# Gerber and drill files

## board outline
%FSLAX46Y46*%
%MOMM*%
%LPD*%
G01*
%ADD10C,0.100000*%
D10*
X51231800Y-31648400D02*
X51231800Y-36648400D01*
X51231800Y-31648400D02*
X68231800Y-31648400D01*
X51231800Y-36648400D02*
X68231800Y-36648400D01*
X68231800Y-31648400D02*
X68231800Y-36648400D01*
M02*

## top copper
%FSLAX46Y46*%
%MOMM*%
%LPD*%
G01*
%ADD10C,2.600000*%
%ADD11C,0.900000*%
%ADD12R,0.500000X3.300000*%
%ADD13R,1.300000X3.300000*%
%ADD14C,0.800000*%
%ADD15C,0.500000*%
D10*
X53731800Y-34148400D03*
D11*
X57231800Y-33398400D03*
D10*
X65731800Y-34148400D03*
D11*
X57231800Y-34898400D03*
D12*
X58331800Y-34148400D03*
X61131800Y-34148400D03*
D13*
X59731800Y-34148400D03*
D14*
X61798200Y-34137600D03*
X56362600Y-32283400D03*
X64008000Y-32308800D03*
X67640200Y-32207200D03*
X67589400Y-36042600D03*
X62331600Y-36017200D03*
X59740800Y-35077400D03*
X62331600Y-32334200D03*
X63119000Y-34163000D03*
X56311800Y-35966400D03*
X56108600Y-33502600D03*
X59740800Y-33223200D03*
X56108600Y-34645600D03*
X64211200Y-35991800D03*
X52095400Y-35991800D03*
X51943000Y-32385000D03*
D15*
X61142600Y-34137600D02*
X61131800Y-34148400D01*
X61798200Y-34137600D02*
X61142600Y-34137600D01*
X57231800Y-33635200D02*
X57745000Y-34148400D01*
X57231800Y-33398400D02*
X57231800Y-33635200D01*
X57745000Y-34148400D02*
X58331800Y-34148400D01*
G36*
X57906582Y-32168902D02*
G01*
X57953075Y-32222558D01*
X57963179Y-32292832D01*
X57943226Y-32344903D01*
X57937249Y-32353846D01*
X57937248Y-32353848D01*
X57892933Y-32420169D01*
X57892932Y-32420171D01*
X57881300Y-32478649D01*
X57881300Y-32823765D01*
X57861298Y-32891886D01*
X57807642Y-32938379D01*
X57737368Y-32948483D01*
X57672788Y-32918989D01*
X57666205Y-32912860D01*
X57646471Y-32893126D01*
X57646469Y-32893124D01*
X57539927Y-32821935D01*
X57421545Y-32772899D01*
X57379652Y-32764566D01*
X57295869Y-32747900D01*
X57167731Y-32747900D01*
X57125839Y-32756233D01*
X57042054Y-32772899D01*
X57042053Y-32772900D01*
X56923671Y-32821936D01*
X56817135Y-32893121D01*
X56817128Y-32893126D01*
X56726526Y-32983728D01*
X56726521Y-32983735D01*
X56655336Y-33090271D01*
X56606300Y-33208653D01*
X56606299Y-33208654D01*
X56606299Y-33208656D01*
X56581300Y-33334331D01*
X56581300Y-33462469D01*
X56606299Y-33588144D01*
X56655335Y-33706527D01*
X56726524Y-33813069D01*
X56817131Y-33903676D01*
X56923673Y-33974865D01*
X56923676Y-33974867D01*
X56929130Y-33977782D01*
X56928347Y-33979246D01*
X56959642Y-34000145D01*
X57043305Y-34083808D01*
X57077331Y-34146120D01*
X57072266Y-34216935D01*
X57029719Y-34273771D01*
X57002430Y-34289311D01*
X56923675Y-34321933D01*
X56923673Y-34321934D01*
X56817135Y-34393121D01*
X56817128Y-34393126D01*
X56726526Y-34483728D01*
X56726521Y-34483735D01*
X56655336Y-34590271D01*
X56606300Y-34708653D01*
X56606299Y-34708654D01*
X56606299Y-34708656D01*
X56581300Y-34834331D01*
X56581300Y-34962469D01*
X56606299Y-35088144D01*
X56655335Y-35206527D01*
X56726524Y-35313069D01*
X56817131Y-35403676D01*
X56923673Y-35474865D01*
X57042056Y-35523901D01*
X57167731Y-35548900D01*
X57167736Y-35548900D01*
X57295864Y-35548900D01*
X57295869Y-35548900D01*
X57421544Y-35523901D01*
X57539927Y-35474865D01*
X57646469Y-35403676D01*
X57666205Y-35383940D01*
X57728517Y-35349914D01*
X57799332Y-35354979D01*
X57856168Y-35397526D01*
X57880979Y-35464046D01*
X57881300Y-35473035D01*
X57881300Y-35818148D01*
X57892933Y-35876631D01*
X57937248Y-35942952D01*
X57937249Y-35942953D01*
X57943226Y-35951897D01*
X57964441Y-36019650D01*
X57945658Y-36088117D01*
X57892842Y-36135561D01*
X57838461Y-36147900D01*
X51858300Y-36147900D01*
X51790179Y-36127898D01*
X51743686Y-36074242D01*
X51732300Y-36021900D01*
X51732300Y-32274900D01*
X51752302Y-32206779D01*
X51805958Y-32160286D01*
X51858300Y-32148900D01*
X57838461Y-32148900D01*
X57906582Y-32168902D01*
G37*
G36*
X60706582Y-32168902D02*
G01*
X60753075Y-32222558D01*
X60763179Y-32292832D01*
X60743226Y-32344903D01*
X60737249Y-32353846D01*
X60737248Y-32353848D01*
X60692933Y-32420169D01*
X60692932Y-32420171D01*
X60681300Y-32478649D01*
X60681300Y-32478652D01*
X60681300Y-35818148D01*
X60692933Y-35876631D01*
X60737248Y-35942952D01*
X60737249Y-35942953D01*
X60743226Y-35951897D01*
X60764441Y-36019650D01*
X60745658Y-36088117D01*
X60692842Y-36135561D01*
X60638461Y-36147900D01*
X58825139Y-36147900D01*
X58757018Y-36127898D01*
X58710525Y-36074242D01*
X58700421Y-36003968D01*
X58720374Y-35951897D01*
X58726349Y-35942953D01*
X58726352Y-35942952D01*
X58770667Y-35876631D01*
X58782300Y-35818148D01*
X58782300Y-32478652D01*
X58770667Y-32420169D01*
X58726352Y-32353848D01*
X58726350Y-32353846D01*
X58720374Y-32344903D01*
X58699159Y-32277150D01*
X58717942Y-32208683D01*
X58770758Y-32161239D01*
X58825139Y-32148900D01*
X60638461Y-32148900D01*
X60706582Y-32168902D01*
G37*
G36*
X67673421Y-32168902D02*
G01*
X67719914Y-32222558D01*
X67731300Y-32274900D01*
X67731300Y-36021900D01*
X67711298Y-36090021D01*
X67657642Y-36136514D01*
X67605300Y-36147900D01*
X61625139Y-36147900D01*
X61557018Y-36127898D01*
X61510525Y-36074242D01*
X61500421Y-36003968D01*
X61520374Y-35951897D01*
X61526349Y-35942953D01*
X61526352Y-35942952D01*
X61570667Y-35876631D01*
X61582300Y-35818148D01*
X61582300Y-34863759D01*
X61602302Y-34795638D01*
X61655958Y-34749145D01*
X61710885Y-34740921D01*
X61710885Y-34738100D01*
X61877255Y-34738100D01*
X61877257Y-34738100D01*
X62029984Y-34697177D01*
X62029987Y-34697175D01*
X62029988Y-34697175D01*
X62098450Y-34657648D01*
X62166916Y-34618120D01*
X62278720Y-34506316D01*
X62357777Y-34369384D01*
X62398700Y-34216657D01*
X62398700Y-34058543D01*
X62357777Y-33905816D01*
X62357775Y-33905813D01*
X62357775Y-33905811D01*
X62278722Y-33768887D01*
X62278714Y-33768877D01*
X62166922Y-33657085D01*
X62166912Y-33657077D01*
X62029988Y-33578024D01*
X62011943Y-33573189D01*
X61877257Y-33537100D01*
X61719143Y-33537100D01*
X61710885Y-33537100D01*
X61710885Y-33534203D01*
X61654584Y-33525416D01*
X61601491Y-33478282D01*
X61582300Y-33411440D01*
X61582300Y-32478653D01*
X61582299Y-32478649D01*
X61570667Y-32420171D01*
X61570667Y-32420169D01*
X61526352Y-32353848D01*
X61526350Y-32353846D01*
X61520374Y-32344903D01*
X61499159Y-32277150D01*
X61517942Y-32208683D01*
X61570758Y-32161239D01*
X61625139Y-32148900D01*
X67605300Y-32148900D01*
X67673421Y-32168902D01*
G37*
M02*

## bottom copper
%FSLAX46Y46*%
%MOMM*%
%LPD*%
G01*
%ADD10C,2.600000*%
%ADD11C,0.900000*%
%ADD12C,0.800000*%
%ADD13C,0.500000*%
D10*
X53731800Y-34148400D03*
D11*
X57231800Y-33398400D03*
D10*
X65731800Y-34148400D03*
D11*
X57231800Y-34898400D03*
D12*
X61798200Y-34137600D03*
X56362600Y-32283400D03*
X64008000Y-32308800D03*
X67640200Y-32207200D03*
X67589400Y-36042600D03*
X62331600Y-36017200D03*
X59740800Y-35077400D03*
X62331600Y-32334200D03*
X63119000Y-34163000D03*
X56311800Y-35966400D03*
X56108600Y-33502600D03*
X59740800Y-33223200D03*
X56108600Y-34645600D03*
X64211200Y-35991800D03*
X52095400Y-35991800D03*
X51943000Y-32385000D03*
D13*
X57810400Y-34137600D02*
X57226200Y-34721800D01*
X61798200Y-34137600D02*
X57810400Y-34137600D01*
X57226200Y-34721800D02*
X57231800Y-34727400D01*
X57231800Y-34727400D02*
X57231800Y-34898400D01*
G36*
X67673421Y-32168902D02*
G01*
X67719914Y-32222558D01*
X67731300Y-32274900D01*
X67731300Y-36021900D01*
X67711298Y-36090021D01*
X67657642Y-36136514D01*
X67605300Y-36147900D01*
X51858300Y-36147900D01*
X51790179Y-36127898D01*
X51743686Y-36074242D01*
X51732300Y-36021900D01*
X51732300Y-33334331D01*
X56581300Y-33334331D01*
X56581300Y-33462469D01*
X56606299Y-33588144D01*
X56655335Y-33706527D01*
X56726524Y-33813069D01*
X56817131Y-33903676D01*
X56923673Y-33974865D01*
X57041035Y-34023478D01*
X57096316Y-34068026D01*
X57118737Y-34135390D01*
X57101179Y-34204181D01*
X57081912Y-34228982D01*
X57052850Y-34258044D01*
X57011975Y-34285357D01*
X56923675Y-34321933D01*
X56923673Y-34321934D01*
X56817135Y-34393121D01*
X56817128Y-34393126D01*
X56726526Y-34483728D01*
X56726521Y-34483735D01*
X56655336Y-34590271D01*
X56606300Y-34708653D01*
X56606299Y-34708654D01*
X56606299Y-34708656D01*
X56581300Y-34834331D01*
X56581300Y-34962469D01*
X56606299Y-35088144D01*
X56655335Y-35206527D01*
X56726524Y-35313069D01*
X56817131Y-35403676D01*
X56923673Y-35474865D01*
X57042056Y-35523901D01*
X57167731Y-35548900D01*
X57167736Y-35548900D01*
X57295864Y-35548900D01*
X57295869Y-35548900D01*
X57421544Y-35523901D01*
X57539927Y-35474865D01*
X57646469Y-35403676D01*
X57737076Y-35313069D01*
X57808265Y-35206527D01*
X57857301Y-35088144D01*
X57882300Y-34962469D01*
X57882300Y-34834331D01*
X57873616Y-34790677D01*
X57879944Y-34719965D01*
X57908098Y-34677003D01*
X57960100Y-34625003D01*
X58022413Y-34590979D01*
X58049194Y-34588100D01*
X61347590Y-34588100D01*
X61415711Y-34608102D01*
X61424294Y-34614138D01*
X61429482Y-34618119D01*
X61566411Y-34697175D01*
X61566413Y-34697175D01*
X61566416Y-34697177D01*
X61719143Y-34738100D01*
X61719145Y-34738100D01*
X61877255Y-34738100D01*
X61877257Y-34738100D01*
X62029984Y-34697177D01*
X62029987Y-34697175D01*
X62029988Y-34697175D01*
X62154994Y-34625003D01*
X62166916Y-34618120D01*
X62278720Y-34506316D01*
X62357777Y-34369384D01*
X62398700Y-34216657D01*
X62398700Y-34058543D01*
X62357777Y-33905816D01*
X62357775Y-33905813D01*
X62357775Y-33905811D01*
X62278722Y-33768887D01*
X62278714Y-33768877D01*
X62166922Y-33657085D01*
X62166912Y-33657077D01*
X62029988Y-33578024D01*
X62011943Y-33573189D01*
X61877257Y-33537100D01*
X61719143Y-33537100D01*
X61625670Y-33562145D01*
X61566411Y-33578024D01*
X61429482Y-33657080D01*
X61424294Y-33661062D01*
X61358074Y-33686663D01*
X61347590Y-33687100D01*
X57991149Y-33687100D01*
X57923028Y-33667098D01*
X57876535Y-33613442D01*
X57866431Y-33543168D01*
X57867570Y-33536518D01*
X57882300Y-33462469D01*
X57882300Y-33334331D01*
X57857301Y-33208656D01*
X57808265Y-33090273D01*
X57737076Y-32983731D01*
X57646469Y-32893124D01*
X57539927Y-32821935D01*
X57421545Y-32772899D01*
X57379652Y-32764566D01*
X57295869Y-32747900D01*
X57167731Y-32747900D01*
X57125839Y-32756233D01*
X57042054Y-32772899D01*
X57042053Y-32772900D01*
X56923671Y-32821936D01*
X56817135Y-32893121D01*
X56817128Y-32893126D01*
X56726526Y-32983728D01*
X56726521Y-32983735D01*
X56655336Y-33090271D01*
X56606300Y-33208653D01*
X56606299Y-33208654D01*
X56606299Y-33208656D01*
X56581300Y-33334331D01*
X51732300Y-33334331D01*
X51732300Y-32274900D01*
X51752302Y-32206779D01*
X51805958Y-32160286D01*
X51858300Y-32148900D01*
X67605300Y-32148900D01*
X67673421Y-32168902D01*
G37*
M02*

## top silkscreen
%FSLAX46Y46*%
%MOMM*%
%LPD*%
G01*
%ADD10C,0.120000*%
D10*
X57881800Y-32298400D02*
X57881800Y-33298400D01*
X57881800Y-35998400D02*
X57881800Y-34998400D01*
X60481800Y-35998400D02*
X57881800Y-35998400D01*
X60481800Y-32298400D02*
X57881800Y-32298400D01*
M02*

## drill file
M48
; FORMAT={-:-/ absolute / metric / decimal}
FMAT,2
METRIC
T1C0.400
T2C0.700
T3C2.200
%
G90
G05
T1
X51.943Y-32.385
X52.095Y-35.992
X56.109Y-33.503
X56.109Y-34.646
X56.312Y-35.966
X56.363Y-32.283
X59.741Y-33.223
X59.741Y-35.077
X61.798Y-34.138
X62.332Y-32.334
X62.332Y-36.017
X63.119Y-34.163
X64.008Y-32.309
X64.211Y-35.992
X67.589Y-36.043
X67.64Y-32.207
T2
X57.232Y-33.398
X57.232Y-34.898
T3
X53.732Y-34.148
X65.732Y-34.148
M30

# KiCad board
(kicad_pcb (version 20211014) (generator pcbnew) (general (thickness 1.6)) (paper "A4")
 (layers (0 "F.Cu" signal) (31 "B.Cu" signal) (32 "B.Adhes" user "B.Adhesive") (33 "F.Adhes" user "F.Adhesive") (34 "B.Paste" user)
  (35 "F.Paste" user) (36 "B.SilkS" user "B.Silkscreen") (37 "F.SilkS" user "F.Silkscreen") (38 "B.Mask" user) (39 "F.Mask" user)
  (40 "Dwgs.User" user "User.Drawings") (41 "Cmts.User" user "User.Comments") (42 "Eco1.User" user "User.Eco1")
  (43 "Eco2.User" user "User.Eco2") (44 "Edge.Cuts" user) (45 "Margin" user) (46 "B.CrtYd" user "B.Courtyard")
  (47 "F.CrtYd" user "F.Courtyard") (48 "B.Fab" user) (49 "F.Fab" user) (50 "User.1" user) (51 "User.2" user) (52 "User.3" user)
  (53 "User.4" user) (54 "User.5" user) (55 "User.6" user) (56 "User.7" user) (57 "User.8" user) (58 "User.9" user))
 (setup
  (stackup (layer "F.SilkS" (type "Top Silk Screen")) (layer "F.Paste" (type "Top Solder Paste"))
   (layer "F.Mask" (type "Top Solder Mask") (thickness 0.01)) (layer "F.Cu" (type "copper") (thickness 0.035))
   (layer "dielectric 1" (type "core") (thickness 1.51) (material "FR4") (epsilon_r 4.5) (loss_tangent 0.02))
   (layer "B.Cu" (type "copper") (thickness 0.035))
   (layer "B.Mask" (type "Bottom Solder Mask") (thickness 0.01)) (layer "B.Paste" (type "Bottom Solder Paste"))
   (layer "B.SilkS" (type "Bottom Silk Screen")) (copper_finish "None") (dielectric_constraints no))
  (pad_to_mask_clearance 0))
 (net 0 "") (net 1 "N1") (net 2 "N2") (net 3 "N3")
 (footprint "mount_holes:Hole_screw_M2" (layer "F.Cu") (at 53.7318 34.1484)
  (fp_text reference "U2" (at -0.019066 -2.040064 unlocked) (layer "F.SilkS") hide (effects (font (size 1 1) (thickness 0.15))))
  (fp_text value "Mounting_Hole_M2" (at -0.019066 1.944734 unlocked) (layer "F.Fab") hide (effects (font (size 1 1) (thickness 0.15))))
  (pad "1" thru_hole circle (at 0 0) (size 2.6 2.6) (drill 2.2) (layers *.Cu *.Mask) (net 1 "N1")))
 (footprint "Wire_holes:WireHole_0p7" (layer "F.Cu") (at 57.2318 33.3984)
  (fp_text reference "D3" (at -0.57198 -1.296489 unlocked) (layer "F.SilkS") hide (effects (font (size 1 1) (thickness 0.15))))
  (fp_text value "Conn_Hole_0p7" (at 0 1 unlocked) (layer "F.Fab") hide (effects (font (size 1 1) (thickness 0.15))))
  (pad "1" thru_hole circle (at 0 0) (size 0.9 0.9) (drill 0.7) (layers *.Cu *.Mask) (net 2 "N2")))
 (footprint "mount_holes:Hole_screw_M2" (layer "F.Cu") (at 65.7318 34.1484)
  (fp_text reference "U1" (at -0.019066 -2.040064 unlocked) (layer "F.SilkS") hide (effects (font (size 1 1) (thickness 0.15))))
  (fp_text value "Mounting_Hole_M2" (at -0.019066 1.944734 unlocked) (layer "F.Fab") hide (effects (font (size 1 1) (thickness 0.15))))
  (pad "1" thru_hole circle (at 0 0) (size 2.6 2.6) (drill 2.2) (layers *.Cu *.Mask) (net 1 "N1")))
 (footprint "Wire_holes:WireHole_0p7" (layer "F.Cu") (at 57.2318 34.8984)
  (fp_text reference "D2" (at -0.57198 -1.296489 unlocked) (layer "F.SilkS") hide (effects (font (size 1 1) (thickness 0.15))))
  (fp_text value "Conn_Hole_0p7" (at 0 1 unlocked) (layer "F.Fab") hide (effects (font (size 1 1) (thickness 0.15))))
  (pad "1" thru_hole circle (at 0 0) (size 0.9 0.9) (drill 0.7) (layers *.Cu *.Mask) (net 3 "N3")))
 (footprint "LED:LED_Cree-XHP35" (layer "F.Cu") (at 59.7318 34.1484)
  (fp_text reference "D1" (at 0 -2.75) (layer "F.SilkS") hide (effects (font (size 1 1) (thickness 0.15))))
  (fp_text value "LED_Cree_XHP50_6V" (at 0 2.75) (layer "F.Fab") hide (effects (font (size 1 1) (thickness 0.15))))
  (fp_line (start -1.85 -1.85) (end -1.85 -0.85) (layer "F.SilkS") (width 0.12))
  (fp_line (start -1.85 1.85) (end -1.85 0.85) (layer "F.SilkS") (width 0.12))
  (fp_line (start 0.75 1.85) (end -1.85 1.85) (layer "F.SilkS") (width 0.12))
  (fp_line (start 0.75 -1.85) (end -1.85 -1.85) (layer "F.SilkS") (width 0.12))
  (pad "" smd rect locked (at 0 1) (size 1.01 0.75) (layers "F.Paste"))
  (pad "" smd rect locked (at 0 -1) (size 1.01 0.75) (layers "F.Paste"))
  (pad "" smd rect locked (at 0 0) (size 1.01 0.75) (layers "F.Paste"))
  (pad "1" smd rect locked (at -1.4 0) (size 0.5 3.3) (layers "F.Cu" "F.Paste" "F.Mask") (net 2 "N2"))
  (pad "2" smd rect locked (at 1.4 0) (size 0.5 3.3) (layers "F.Cu" "F.Paste" "F.Mask") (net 3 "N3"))
  (pad "3" smd rect locked (at 0 0) (size 1.3 3.3) (layers "F.Cu" "F.Mask") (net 1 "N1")))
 (gr_line (start 51.2318 31.6484) (end 51.2318 36.6484) (layer "Edge.Cuts") (width 0.1))
 (gr_line (start 51.2318 31.6484) (end 68.2318 31.6484) (layer "Edge.Cuts") (width 0.1))
 (gr_line (start 51.2318 36.6484) (end 68.2318 36.6484) (layer "Edge.Cuts") (width 0.1))
 (gr_line (start 68.2318 31.6484) (end 68.2318 36.6484) (layer "Edge.Cuts") (width 0.1))
 (segment (start 61.1426 34.1376) (end 61.1318 34.1484) (width 0.5) (layer "F.Cu") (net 3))
 (segment (start 61.7982 34.1376) (end 61.1426 34.1376) (width 0.5) (layer "F.Cu") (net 3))
 (via (at 61.7982 34.1376) (size 0.8) (drill 0.4) (layers "F.Cu" "B.Cu") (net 3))
 (segment (start 57.8104 34.1376) (end 57.2262 34.7218) (width 0.5) (layer "B.Cu") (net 3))
 (segment (start 61.7982 34.1376) (end 57.8104 34.1376) (width 0.5) (layer "B.Cu") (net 3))
 (segment (start 57.2262 34.7218) (end 57.2318 34.7274) (width 0.5) (layer "B.Cu") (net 3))
 (segment (start 57.2318 34.7274) (end 57.2318 34.8984) (width 0.5) (layer "B.Cu") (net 3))
 (segment (start 57.2318 33.6352) (end 57.745 34.1484) (width 0.5) (layer "F.Cu") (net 2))
 (segment (start 57.2318 33.3984) (end 57.2318 33.6352) (width 0.5) (layer "F.Cu") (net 2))
 (segment (start 57.745 34.1484) (end 58.3318 34.1484) (width 0.5) (layer "F.Cu") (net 2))
 (via (at 56.3626 32.2834) (size 0.8) (drill 0.4) (layers "F.Cu" "B.Cu") (free) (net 1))
 (via (at 64.008 32.3088) (size 0.8) (drill 0.4) (layers "F.Cu" "B.Cu") (free) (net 1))
 (via (at 67.6402 32.2072) (size 0.8) (drill 0.4) (layers "F.Cu" "B.Cu") (free) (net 1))
 (via (at 67.5894 36.0426) (size 0.8) (drill 0.4) (layers "F.Cu" "B.Cu") (free) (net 1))
 (via (at 62.3316 36.0172) (size 0.8) (drill 0.4) (layers "F.Cu" "B.Cu") (free) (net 1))
 (via (at 59.7408 35.0774) (size 0.8) (drill 0.4) (layers "F.Cu" "B.Cu") (free) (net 1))
 (via (at 62.3316 32.3342) (size 0.8) (drill 0.4) (layers "F.Cu" "B.Cu") (free) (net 1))
 (via (at 63.119 34.163) (size 0.8) (drill 0.4) (layers "F.Cu" "B.Cu") (free) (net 1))
 (via (at 56.3118 35.9664) (size 0.8) (drill 0.4) (layers "F.Cu" "B.Cu") (free) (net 1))
 (via (at 56.1086 33.5026) (size 0.8) (drill 0.4) (layers "F.Cu" "B.Cu") (free) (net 1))
 (via (at 59.7408 33.2232) (size 0.8) (drill 0.4) (layers "F.Cu" "B.Cu") (free) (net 1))
 (via (at 56.1086 34.6456) (size 0.8) (drill 0.4) (layers "F.Cu" "B.Cu") (free) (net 1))
 (via (at 64.2112 35.9918) (size 0.8) (drill 0.4) (layers "F.Cu" "B.Cu") (free) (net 1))
 (via (at 52.0954 35.9918) (size 0.8) (drill 0.4) (layers "F.Cu" "B.Cu") (free) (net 1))
 (via (at 51.943 32.385) (size 0.8) (drill 0.4) (layers "F.Cu" "B.Cu") (free) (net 1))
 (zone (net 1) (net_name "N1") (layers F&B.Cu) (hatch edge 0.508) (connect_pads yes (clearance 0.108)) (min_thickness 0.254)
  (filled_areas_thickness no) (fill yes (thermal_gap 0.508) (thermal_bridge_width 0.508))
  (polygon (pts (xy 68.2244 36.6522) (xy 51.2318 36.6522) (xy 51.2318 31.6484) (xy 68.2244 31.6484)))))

